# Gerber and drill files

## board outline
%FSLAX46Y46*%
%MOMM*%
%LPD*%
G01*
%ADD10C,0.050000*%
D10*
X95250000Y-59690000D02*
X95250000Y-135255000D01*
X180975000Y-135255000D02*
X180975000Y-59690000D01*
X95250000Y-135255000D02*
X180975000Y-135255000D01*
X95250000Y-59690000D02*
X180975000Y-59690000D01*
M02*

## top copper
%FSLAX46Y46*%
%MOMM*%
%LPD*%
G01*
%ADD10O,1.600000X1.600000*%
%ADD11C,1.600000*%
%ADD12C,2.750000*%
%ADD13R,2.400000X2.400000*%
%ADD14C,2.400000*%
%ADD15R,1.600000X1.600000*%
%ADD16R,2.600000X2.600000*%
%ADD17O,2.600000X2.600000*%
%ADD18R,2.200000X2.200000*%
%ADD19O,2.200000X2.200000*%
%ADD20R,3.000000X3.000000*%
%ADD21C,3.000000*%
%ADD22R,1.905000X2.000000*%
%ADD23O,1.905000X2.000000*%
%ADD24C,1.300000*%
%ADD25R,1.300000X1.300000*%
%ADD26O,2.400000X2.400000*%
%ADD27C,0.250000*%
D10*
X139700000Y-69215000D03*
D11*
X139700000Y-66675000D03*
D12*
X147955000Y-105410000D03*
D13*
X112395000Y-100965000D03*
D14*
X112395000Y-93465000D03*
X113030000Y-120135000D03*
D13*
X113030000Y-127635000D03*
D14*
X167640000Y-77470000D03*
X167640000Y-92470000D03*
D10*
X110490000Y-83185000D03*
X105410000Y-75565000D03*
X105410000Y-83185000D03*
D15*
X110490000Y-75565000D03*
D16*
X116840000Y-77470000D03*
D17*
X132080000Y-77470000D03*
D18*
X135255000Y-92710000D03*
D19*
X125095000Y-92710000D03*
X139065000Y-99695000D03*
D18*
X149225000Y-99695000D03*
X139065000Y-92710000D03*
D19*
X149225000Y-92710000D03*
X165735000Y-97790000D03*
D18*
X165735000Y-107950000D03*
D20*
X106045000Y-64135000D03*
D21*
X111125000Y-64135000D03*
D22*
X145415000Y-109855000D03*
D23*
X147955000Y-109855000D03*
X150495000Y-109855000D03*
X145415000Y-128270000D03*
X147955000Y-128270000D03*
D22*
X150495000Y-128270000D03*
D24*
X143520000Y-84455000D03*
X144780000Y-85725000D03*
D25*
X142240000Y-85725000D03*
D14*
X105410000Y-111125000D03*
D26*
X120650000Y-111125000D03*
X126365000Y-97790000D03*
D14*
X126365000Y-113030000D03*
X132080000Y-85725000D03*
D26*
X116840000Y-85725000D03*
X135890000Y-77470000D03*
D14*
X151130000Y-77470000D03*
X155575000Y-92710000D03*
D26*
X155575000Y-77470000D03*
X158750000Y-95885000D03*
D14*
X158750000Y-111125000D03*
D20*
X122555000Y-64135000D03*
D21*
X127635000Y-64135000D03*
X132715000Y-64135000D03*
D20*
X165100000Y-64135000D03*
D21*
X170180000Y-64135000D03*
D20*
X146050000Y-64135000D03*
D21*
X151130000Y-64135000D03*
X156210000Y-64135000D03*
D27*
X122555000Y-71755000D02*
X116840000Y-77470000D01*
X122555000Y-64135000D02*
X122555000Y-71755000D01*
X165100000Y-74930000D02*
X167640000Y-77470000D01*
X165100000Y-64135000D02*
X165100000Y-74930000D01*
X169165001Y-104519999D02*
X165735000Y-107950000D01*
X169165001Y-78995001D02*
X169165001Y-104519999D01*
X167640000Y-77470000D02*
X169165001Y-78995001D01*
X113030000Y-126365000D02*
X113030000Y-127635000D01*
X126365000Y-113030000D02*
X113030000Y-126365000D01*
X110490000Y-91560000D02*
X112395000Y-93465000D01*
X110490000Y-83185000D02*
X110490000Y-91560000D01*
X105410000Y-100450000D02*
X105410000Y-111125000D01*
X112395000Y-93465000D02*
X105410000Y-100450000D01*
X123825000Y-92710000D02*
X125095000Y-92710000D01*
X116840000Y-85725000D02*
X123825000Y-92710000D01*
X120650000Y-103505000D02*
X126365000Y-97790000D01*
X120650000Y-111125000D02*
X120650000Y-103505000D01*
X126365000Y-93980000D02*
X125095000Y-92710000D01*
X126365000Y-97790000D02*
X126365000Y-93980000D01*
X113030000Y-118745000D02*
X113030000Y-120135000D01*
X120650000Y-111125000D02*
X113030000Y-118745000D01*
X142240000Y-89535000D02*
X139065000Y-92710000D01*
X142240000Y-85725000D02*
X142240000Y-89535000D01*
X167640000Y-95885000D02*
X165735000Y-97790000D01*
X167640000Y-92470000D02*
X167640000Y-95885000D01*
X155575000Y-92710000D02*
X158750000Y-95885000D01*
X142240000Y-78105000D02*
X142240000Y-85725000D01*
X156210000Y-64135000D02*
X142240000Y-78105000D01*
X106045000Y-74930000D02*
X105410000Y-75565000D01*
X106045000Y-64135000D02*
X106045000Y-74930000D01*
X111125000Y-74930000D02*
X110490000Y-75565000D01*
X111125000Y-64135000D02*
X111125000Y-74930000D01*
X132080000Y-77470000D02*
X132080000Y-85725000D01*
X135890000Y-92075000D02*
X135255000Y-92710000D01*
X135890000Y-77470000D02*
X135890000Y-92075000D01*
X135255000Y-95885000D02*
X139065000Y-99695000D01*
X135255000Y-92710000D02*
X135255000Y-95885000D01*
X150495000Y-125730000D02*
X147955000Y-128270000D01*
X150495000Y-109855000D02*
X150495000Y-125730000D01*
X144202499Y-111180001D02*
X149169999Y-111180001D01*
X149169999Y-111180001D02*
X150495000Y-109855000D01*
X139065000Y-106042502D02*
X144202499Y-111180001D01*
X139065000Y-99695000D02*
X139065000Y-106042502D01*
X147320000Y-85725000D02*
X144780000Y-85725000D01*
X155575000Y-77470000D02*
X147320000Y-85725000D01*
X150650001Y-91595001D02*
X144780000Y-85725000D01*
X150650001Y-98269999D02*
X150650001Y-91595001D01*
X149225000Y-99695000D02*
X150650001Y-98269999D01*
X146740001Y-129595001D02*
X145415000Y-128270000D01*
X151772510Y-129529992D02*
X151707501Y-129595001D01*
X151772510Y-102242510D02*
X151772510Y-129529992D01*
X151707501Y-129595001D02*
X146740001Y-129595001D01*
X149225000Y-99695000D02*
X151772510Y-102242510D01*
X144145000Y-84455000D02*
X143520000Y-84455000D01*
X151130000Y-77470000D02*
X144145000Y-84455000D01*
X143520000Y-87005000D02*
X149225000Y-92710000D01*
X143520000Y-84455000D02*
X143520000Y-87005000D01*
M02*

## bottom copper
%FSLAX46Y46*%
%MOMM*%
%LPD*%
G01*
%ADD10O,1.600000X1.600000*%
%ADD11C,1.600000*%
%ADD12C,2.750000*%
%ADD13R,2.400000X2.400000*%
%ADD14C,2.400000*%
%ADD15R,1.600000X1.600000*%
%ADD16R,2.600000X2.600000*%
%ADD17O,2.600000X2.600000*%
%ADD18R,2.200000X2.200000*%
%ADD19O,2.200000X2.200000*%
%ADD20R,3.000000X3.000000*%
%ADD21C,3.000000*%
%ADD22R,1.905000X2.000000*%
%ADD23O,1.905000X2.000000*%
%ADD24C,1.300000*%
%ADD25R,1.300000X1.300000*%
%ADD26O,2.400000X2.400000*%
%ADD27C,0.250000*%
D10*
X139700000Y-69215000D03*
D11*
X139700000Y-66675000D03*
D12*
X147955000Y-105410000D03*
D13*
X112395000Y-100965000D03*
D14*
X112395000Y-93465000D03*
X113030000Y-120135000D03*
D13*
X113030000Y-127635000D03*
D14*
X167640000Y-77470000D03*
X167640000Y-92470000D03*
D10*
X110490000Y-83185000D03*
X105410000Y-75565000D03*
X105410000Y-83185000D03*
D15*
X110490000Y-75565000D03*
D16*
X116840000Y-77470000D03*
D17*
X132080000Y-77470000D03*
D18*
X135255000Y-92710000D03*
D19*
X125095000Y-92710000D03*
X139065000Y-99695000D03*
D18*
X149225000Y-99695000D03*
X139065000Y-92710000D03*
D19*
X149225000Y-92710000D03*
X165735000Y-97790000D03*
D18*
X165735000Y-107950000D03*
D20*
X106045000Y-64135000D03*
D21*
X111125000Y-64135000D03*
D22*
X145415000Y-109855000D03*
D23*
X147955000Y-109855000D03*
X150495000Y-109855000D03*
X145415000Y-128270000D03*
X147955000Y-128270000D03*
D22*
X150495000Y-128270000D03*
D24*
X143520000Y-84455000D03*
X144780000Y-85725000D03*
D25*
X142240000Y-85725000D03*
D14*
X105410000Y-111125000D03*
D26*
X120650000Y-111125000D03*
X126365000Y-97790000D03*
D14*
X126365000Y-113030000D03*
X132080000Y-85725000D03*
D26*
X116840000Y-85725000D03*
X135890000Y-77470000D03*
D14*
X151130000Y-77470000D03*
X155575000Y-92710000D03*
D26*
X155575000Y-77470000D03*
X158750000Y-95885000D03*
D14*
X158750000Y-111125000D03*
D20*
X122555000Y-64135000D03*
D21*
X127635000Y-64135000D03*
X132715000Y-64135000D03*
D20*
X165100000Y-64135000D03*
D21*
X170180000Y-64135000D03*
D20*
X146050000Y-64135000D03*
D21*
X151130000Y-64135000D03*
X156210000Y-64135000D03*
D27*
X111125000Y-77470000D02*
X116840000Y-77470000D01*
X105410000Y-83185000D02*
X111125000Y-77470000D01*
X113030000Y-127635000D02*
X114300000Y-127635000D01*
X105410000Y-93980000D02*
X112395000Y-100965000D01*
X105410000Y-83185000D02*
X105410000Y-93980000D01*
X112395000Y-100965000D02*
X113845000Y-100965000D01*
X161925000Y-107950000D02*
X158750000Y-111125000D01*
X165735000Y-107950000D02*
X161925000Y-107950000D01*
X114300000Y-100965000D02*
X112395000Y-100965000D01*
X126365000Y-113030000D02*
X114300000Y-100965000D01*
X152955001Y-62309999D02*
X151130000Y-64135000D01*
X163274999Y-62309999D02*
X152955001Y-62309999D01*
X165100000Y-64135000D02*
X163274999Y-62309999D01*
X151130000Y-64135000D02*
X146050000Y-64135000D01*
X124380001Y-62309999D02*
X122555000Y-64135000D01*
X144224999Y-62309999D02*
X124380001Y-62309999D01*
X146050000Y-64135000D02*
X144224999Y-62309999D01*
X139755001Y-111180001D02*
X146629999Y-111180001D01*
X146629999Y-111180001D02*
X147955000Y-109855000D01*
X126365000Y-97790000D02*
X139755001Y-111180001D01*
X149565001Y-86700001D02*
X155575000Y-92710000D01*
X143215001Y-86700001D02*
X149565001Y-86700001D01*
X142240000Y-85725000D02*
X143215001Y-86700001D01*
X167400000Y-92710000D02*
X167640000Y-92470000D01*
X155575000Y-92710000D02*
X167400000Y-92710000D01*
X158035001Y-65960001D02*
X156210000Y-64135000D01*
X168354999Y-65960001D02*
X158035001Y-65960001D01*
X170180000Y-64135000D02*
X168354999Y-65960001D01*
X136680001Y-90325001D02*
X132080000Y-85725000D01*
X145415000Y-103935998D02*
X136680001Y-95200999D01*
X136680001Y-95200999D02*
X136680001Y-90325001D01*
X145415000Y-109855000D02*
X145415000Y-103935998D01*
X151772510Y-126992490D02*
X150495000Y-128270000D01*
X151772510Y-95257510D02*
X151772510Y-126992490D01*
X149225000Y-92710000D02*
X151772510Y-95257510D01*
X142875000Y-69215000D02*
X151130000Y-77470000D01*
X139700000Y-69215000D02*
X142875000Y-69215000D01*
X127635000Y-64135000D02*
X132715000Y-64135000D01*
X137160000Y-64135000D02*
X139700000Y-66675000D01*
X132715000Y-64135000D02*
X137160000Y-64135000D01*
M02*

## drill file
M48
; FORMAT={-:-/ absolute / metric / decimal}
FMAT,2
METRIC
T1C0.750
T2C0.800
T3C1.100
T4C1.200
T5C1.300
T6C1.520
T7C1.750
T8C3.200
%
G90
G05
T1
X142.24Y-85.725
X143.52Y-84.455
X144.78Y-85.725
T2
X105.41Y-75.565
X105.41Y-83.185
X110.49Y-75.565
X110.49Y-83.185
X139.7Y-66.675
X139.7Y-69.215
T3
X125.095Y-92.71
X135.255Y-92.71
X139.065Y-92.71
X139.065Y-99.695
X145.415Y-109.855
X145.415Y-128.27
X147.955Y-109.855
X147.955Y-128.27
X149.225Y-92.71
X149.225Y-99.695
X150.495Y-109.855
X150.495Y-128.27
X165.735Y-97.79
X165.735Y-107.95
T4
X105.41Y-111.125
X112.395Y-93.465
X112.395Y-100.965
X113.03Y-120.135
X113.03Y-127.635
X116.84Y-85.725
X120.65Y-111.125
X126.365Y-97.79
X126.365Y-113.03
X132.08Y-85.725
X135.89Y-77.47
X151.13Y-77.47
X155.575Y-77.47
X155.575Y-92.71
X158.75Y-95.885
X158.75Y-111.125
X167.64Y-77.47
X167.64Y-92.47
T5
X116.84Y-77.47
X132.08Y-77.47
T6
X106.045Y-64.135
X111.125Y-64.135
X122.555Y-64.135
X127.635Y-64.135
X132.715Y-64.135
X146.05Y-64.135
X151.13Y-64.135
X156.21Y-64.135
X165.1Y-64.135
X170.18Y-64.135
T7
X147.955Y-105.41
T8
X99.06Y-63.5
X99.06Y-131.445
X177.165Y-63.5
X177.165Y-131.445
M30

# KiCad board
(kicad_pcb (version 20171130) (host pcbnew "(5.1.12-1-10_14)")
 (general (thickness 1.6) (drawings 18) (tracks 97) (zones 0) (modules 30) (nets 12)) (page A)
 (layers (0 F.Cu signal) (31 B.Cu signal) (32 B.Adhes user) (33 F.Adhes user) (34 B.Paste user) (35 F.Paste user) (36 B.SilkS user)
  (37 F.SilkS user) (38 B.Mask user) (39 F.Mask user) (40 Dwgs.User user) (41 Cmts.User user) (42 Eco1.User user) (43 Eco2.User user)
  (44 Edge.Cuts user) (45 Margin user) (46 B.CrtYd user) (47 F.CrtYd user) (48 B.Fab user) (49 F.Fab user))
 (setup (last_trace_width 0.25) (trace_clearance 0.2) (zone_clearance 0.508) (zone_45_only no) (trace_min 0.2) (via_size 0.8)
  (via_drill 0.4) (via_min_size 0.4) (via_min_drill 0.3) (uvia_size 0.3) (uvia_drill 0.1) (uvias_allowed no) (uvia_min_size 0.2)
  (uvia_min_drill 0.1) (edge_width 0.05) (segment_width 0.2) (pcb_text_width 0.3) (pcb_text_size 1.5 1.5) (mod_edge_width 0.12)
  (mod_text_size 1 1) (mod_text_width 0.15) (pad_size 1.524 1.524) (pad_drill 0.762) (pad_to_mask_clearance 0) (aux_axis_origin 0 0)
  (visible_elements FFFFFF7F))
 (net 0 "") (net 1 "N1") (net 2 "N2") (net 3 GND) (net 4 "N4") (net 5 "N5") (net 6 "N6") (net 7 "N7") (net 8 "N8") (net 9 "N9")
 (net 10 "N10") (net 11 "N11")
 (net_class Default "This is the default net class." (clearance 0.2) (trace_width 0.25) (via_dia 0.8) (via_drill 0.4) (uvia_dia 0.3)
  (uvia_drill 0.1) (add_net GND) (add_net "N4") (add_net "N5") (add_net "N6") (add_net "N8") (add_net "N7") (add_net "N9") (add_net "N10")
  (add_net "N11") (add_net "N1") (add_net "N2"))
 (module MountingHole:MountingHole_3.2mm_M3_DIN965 (layer F.Cu) (at 177.165 131.445)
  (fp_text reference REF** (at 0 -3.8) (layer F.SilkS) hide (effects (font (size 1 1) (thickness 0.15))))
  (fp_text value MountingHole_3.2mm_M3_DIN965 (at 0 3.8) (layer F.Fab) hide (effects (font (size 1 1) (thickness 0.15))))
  (pad 1 np_thru_hole circle (at 0 0) (size 3.2 3.2) (drill 3.2) (layers *.Cu *.Mask)))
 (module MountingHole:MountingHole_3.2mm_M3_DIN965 (layer F.Cu) (at 99.06 131.445)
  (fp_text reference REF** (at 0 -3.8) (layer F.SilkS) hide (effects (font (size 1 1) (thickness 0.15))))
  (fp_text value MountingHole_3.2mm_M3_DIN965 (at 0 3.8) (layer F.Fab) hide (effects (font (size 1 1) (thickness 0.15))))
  (pad 1 np_thru_hole circle (at 0 0) (size 3.2 3.2) (drill 3.2) (layers *.Cu *.Mask)))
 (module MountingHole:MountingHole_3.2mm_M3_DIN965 (layer F.Cu) (at 99.06 63.5)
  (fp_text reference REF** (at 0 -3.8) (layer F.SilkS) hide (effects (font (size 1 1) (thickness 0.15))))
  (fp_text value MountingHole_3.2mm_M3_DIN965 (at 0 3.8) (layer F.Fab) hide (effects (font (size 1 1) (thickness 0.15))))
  (pad 1 np_thru_hole circle (at 0 0) (size 3.2 3.2) (drill 3.2) (layers *.Cu *.Mask)))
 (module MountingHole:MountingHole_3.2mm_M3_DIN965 (layer F.Cu) (at 177.165 63.5)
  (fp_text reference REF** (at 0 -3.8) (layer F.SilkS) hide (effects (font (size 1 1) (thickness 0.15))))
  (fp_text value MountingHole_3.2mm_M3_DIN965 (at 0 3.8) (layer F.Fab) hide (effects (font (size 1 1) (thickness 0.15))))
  (pad 1 np_thru_hole circle (at 0 0) (size 3.2 3.2) (drill 3.2) (layers *.Cu *.Mask)))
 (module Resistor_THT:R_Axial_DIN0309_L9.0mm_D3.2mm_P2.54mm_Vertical (layer F.Cu) (at 139.7 66.675 270)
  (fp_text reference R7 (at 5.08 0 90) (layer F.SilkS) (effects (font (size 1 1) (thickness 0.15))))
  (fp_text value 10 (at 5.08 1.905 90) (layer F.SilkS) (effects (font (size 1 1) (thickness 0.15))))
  (pad 2 thru_hole oval (at 2.54 0 270) (size 1.6 1.6) (drill 0.8) (layers *.Cu *.Mask) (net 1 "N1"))
  (pad 1 thru_hole circle (at 0 0 270) (size 1.6 1.6) (drill 0.8) (layers *.Cu *.Mask) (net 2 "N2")))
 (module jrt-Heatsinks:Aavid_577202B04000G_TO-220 (layer F.Cu) (at 147.955 105.41 180)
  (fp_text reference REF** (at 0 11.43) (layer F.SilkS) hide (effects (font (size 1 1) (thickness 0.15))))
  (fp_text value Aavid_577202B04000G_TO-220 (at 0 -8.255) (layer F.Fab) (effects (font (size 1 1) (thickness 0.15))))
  (pad "" thru_hole circle (at 0 0 180) (size 2.75 2.75) (drill 1.75) (layers *.Cu *.Mask)))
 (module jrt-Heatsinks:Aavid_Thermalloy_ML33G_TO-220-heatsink (layer F.Cu) (at 167.005 135.255 180)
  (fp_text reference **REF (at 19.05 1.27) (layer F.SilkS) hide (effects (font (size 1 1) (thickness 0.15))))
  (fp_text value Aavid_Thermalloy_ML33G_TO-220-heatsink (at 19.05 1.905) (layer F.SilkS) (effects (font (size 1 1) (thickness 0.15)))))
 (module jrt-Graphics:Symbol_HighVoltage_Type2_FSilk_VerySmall (layer F.Cu) (at 168.91 112.395 90)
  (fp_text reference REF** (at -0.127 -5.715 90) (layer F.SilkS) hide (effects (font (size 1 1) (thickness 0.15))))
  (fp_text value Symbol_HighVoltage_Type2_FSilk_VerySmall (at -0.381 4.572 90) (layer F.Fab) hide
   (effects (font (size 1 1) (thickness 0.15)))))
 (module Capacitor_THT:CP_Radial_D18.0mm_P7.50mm (layer F.Cu) (at 112.395 100.965 90)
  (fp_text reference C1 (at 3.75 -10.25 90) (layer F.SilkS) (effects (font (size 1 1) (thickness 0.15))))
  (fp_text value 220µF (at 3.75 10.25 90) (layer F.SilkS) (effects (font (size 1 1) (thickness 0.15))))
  (pad 1 thru_hole rect (at 0 0 90) (size 2.4 2.4) (drill 1.2) (layers *.Cu *.Mask) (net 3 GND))
  (pad 2 thru_hole circle (at 7.5 0 90) (size 2.4 2.4) (drill 1.2) (layers *.Cu *.Mask) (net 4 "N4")))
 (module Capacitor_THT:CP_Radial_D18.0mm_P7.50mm (layer F.Cu) (at 113.03 127.635 90)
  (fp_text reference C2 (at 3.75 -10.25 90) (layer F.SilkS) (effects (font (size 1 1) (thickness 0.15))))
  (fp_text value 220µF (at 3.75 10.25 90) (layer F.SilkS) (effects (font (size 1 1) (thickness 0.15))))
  (pad 2 thru_hole circle (at 7.5 0 90) (size 2.4 2.4) (drill 1.2) (layers *.Cu *.Mask) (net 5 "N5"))
  (pad 1 thru_hole rect (at 0 0 90) (size 2.4 2.4) (drill 1.2) (layers *.Cu *.Mask) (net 3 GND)))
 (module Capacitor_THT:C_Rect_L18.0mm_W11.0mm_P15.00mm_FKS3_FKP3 (layer F.Cu) (at 167.64 77.47 270)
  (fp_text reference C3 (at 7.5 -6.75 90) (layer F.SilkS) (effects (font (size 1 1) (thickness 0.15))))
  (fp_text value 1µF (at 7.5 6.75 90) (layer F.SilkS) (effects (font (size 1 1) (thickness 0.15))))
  (pad 1 thru_hole circle (at 0 0 270) (size 2.4 2.4) (drill 1.2) (layers *.Cu *.Mask) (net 3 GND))
  (pad 2 thru_hole circle (at 15 0 270) (size 2.4 2.4) (drill 1.2) (layers *.Cu *.Mask) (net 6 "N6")))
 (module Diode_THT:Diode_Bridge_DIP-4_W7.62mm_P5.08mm (layer F.Cu) (at 110.49 75.565 270)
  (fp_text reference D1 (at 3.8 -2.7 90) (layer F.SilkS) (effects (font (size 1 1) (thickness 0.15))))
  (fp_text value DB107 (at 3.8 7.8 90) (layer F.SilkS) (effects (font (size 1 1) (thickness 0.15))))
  (pad 4 thru_hole oval (at 7.62 0 270) (size 1.6 1.6) (drill 0.8) (layers *.Cu *.Mask) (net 4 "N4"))
  (pad 2 thru_hole oval (at 0 5.08 270) (size 1.6 1.6) (drill 0.8) (layers *.Cu *.Mask) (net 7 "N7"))
  (pad 3 thru_hole oval (at 7.62 5.08 270) (size 1.6 1.6) (drill 0.8) (layers *.Cu *.Mask) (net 3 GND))
  (pad 1 thru_hole rect (at 0 0 270) (size 1.6 1.6) (drill 0.8) (layers *.Cu *.Mask) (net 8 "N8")))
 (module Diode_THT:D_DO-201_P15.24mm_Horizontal (layer F.Cu) (at 116.84 77.47)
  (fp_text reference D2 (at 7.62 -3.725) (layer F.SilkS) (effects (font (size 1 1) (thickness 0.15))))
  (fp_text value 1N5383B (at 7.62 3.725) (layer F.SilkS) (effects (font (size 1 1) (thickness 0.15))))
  (pad 1 thru_hole rect (at 0 0) (size 2.6 2.6) (drill 1.3) (layers *.Cu *.Mask) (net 3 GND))
  (pad 2 thru_hole oval (at 15.24 0) (size 2.6 2.6) (drill 1.3) (layers *.Cu *.Mask) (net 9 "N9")))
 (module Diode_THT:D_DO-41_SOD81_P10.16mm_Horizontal (layer F.Cu) (at 135.255 92.71 180)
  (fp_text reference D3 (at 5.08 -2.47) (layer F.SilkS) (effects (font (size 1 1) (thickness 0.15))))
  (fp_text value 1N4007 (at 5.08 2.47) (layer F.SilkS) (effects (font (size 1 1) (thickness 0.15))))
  (pad 1 thru_hole rect (at 0 0 180) (size 2.2 2.2) (drill 1.1) (layers *.Cu *.Mask) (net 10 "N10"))
  (pad 2 thru_hole oval (at 10.16 0 180) (size 2.2 2.2) (drill 1.1) (layers *.Cu *.Mask) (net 5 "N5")))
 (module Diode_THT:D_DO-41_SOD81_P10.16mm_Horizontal (layer F.Cu) (at 149.225 99.695 180)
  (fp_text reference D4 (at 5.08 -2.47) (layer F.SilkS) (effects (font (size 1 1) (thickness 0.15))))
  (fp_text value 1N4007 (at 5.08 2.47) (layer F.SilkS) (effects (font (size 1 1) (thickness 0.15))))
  (pad 2 thru_hole oval (at 10.16 0 180) (size 2.2 2.2) (drill 1.1) (layers *.Cu *.Mask) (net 10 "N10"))
  (pad 1 thru_hole rect (at 0 0 180) (size 2.2 2.2) (drill 1.1) (layers *.Cu *.Mask) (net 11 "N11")))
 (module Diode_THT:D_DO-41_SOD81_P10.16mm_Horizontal (layer F.Cu) (at 139.065 92.71)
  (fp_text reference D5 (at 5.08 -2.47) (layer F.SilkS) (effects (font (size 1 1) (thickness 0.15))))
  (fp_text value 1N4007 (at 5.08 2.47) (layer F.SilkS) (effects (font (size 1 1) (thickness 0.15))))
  (pad 1 thru_hole rect (at 0 0) (size 2.2 2.2) (drill 1.1) (layers *.Cu *.Mask) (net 6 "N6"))
  (pad 2 thru_hole oval (at 10.16 0) (size 2.2 2.2) (drill 1.1) (layers *.Cu *.Mask) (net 1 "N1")))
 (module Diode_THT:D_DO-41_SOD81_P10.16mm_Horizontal (layer F.Cu) (at 165.735 107.95 90)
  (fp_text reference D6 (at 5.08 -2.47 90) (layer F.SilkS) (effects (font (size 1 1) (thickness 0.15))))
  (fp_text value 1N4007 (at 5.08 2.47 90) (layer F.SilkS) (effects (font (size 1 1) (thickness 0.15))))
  (pad 2 thru_hole oval (at 10.16 0 90) (size 2.2 2.2) (drill 1.1) (layers *.Cu *.Mask) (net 6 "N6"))
  (pad 1 thru_hole rect (at 0 0 90) (size 2.2 2.2) (drill 1.1) (layers *.Cu *.Mask) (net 3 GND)))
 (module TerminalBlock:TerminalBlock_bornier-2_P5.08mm (layer F.Cu) (at 106.045 64.135)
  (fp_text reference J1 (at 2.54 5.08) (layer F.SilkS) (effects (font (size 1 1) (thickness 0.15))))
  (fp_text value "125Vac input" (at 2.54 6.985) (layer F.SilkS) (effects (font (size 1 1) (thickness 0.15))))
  (pad 1 thru_hole rect (at 0 0) (size 3 3) (drill 1.52) (layers *.Cu *.Mask) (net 7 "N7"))
  (pad 2 thru_hole circle (at 5.08 0) (size 3 3) (drill 1.52) (layers *.Cu *.Mask) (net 8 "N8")))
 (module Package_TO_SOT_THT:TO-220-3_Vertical (layer F.Cu) (at 145.415 109.855)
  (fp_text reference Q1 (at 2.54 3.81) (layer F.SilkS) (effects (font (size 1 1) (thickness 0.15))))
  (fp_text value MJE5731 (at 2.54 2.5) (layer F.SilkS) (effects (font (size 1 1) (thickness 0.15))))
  (pad 1 thru_hole rect (at 0 0) (size 1.905 2) (drill 1.1) (layers *.Cu *.Mask) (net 9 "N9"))
  (pad 2 thru_hole oval (at 2.54 0) (size 1.905 2) (drill 1.1) (layers *.Cu *.Mask) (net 5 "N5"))
  (pad 3 thru_hole oval (at 5.08 0) (size 1.905 2) (drill 1.1) (layers *.Cu *.Mask) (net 10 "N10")))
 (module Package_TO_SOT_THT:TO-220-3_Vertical (layer F.Cu) (at 150.495 128.27 180)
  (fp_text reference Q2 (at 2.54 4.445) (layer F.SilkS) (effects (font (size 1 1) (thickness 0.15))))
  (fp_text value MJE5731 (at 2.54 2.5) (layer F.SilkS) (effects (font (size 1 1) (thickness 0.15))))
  (pad 3 thru_hole oval (at 5.08 0 180) (size 1.905 2) (drill 1.1) (layers *.Cu *.Mask) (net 11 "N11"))
  (pad 2 thru_hole oval (at 2.54 0 180) (size 1.905 2) (drill 1.1) (layers *.Cu *.Mask) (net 10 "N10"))
  (pad 1 thru_hole rect (at 0 0 180) (size 1.905 2) (drill 1.1) (layers *.Cu *.Mask) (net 1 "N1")))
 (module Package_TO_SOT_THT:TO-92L (layer F.Cu) (at 142.24 85.725)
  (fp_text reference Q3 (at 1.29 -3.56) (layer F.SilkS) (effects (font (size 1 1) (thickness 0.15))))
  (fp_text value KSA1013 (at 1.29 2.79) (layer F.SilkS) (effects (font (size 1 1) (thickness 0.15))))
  (pad 2 thru_hole circle (at 1.28 -1.27) (size 1.3 1.3) (drill 0.75) (layers *.Cu *.Mask) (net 1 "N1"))
  (pad 3 thru_hole circle (at 2.54 0) (size 1.3 1.3) (drill 0.75) (layers *.Cu *.Mask) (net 11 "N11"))
  (pad 1 thru_hole rect (at 0 0) (size 1.3 1.3) (drill 0.75) (layers *.Cu *.Mask) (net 6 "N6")))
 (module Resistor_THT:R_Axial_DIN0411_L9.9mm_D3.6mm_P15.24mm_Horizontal (layer F.Cu) (at 105.41 111.125)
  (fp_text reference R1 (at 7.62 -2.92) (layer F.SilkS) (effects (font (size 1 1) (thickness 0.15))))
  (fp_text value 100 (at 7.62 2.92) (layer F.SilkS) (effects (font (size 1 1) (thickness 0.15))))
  (pad 1 thru_hole circle (at 0 0) (size 2.4 2.4) (drill 1.2) (layers *.Cu *.Mask) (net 4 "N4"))
  (pad 2 thru_hole oval (at 15.24 0) (size 2.4 2.4) (drill 1.2) (layers *.Cu *.Mask) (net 5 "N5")))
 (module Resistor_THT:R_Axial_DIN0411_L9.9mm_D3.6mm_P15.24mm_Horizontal (layer F.Cu) (at 126.365 113.03 90)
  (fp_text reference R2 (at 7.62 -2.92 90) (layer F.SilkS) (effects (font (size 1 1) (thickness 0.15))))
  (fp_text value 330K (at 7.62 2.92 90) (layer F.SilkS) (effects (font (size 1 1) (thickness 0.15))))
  (pad 2 thru_hole oval (at 15.24 0 90) (size 2.4 2.4) (drill 1.2) (layers *.Cu *.Mask) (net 5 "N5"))
  (pad 1 thru_hole circle (at 0 0 90) (size 2.4 2.4) (drill 1.2) (layers *.Cu *.Mask) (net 3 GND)))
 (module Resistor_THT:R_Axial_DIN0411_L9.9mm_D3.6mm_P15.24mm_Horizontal (layer F.Cu) (at 132.08 85.725 180)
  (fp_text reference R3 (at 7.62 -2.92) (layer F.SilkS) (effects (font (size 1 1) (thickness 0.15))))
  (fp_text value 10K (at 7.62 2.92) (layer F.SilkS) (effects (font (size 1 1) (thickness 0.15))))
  (pad 1 thru_hole circle (at 0 0 180) (size 2.4 2.4) (drill 1.2) (layers *.Cu *.Mask) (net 9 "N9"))
  (pad 2 thru_hole oval (at 15.24 0 180) (size 2.4 2.4) (drill 1.2) (layers *.Cu *.Mask) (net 5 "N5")))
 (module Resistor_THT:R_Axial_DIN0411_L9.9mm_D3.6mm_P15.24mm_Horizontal (layer F.Cu) (at 151.13 77.47 180)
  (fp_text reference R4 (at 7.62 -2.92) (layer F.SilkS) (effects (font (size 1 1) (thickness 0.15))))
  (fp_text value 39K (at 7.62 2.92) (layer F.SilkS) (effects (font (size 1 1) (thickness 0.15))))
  (pad 2 thru_hole oval (at 15.24 0 180) (size 2.4 2.4) (drill 1.2) (layers *.Cu *.Mask) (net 10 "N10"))
  (pad 1 thru_hole circle (at 0 0 180) (size 2.4 2.4) (drill 1.2) (layers *.Cu *.Mask) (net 1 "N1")))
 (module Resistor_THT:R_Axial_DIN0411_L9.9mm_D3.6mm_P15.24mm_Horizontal (layer F.Cu) (at 155.575 92.71 90)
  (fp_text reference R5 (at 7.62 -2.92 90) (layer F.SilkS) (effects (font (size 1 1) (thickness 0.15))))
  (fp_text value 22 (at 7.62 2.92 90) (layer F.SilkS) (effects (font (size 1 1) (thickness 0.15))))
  (pad 1 thru_hole circle (at 0 0 90) (size 2.4 2.4) (drill 1.2) (layers *.Cu *.Mask) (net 6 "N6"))
  (pad 2 thru_hole oval (at 15.24 0 90) (size 2.4 2.4) (drill 1.2) (layers *.Cu *.Mask) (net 11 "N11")))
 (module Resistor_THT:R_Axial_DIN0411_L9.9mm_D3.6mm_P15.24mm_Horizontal (layer F.Cu) (at 158.75 111.125 90)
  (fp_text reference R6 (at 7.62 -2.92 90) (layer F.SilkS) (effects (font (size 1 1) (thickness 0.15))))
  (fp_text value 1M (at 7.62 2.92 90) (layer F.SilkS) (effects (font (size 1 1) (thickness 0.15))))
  (pad 2 thru_hole oval (at 15.24 0 90) (size 2.4 2.4) (drill 1.2) (layers *.Cu *.Mask) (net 6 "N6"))
  (pad 1 thru_hole circle (at 0 0 90) (size 2.4 2.4) (drill 1.2) (layers *.Cu *.Mask) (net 3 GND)))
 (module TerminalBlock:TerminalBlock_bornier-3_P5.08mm (layer F.Cu) (at 122.555 64.135)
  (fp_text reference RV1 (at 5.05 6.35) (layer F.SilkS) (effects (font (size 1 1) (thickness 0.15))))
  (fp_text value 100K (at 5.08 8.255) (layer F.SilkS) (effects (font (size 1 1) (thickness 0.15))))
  (pad 1 thru_hole rect (at 0 0) (size 3 3) (drill 1.52) (layers *.Cu *.Mask) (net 3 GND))
  (pad 2 thru_hole circle (at 5.08 0) (size 3 3) (drill 1.52) (layers *.Cu *.Mask) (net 2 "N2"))
  (pad 3 thru_hole circle (at 10.16 0) (size 3 3) (drill 1.52) (layers *.Cu *.Mask) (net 2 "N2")))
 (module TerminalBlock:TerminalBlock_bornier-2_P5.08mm (layer F.Cu) (at 165.1 64.135)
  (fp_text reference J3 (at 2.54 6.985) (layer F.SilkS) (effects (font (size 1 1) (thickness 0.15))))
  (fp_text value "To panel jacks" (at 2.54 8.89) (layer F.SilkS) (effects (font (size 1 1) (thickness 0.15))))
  (pad 1 thru_hole rect (at 0 0) (size 3 3) (drill 1.52) (layers *.Cu *.Mask) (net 3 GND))
  (pad 2 thru_hole circle (at 5.08 0) (size 3 3) (drill 1.52) (layers *.Cu *.Mask) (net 6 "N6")))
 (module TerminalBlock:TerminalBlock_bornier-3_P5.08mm (layer F.Cu) (at 146.05 64.135)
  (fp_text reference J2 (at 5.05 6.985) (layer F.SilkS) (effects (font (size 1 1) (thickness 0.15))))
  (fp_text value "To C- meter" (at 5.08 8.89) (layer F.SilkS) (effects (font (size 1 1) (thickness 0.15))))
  (pad 1 thru_hole rect (at 0 0) (size 3 3) (drill 1.52) (layers *.Cu *.Mask) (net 3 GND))
  (pad 2 thru_hole circle (at 5.08 0) (size 3 3) (drill 1.52) (layers *.Cu *.Mask) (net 3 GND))
  (pad 3 thru_hole circle (at 10.16 0) (size 3 3) (drill 1.52) (layers *.Cu *.Mask) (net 6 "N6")))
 (gr_line (start 95.25 59.69) (end 95.25 135.255) (layer Edge.Cuts) (width 0.05))
 (gr_line (start 180.975 135.255) (end 180.975 59.69) (layer Edge.Cuts) (width 0.05))
 (gr_line (start 95.25 135.255) (end 180.975 135.255) (layer Edge.Cuts) (width 0.05))
 (gr_line (start 95.25 59.69) (end 180.975 59.69) (layer Edge.Cuts) (width 0.05))
 (segment (start 122.555 71.755) (end 116.84 77.47) (width 0.25) (layer F.Cu) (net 3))
 (segment (start 122.555 64.135) (end 122.555 71.755) (width 0.25) (layer F.Cu) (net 3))
 (segment (start 111.125 77.47) (end 116.84 77.47) (width 0.25) (layer B.Cu) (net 3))
 (segment (start 105.41 83.185) (end 111.125 77.47) (width 0.25) (layer B.Cu) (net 3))
 (segment (start 165.1 74.93) (end 167.64 77.47) (width 0.25) (layer F.Cu) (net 3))
 (segment (start 165.1 64.135) (end 165.1 74.93) (width 0.25) (layer F.Cu) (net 3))
 (segment (start 113.03 127.635) (end 114.3 127.635) (width 0.25) (layer B.Cu) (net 3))
 (segment (start 105.41 93.98) (end 112.395 100.965) (width 0.25) (layer B.Cu) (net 3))
 (segment (start 105.41 83.185) (end 105.41 93.98) (width 0.25) (layer B.Cu) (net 3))
 (segment (start 112.395 100.965) (end 113.845 100.965) (width 0.25) (layer B.Cu) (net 3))
 (segment (start 169.165001 104.519999) (end 165.735 107.95) (width 0.25) (layer F.Cu) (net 3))
 (segment (start 169.165001 78.995001) (end 169.165001 104.519999) (width 0.25) (layer F.Cu) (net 3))
 (segment (start 167.64 77.47) (end 169.165001 78.995001) (width 0.25) (layer F.Cu) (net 3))
 (segment (start 161.925 107.95) (end 158.75 111.125) (width 0.25) (layer B.Cu) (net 3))
 (segment (start 165.735 107.95) (end 161.925 107.95) (width 0.25) (layer B.Cu) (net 3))
 (segment (start 114.3 100.965) (end 112.395 100.965) (width 0.25) (layer B.Cu) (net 3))
 (segment (start 126.365 113.03) (end 114.3 100.965) (width 0.25) (layer B.Cu) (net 3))
 (segment (start 113.03 126.365) (end 113.03 127.635) (width 0.25) (layer F.Cu) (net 3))
 (segment (start 126.365 113.03) (end 113.03 126.365) (width 0.25) (layer F.Cu) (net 3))
 (segment (start 152.955001 62.309999) (end 151.13 64.135) (width 0.25) (layer B.Cu) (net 3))
 (segment (start 163.274999 62.309999) (end 152.955001 62.309999) (width 0.25) (layer B.Cu) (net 3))
 (segment (start 165.1 64.135) (end 163.274999 62.309999) (width 0.25) (layer B.Cu) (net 3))
 (segment (start 151.13 64.135) (end 146.05 64.135) (width 0.25) (layer B.Cu) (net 3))
 (segment (start 124.380001 62.309999) (end 122.555 64.135) (width 0.25) (layer B.Cu) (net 3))
 (segment (start 144.224999 62.309999) (end 124.380001 62.309999) (width 0.25) (layer B.Cu) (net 3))
 (segment (start 146.05 64.135) (end 144.224999 62.309999) (width 0.25) (layer B.Cu) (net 3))
 (segment (start 110.49 91.56) (end 112.395 93.465) (width 0.25) (layer F.Cu) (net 4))
 (segment (start 110.49 83.185) (end 110.49 91.56) (width 0.25) (layer F.Cu) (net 4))
 (segment (start 105.41 100.45) (end 105.41 111.125) (width 0.25) (layer F.Cu) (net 4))
 (segment (start 112.395 93.465) (end 105.41 100.45) (width 0.25) (layer F.Cu) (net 4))
 (segment (start 123.825 92.71) (end 125.095 92.71) (width 0.25) (layer F.Cu) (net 5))
 (segment (start 116.84 85.725) (end 123.825 92.71) (width 0.25) (layer F.Cu) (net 5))
 (segment (start 120.65 103.505) (end 126.365 97.79) (width 0.25) (layer F.Cu) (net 5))
 (segment (start 120.65 111.125) (end 120.65 103.505) (width 0.25) (layer F.Cu) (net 5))
 (segment (start 126.365 93.98) (end 125.095 92.71) (width 0.25) (layer F.Cu) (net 5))
 (segment (start 126.365 97.79) (end 126.365 93.98) (width 0.25) (layer F.Cu) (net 5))
 (segment (start 139.755001 111.180001) (end 146.629999 111.180001) (width 0.25) (layer B.Cu) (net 5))
 (segment (start 146.629999 111.180001) (end 147.955 109.855) (width 0.25) (layer B.Cu) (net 5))
 (segment (start 126.365 97.79) (end 139.755001 111.180001) (width 0.25) (layer B.Cu) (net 5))
 (segment (start 113.03 118.745) (end 113.03 120.135) (width 0.25) (layer F.Cu) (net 5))
 (segment (start 120.65 111.125) (end 113.03 118.745) (width 0.25) (layer F.Cu) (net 5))
 (segment (start 142.24 89.535) (end 139.065 92.71) (width 0.25) (layer F.Cu) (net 6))
 (segment (start 142.24 85.725) (end 142.24 89.535) (width 0.25) (layer F.Cu) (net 6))
 (segment (start 149.565001 86.700001) (end 155.575 92.71) (width 0.25) (layer B.Cu) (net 6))
 (segment (start 143.215001 86.700001) (end 149.565001 86.700001) (width 0.25) (layer B.Cu) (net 6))
 (segment (start 142.24 85.725) (end 143.215001 86.700001) (width 0.25) (layer B.Cu) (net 6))
 (segment (start 167.4 92.71) (end 167.64 92.47) (width 0.25) (layer B.Cu) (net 6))
 (segment (start 155.575 92.71) (end 167.4 92.71) (width 0.25) (layer B.Cu) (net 6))
 (segment (start 167.64 95.885) (end 165.735 97.79) (width 0.25) (layer F.Cu) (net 6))
 (segment (start 167.64 92.47) (end 167.64 95.885) (width 0.25) (layer F.Cu) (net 6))
 (segment (start 155.575 92.71) (end 158.75 95.885) (width 0.25) (layer F.Cu) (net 6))
 (segment (start 142.24 78.105) (end 142.24 85.725) (width 0.25) (layer F.Cu) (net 6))
 (segment (start 156.21 64.135) (end 142.24 78.105) (width 0.25) (layer F.Cu) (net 6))
 (segment (start 158.035001 65.960001) (end 156.21 64.135) (width 0.25) (layer B.Cu) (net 6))
 (segment (start 168.354999 65.960001) (end 158.035001 65.960001) (width 0.25) (layer B.Cu) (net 6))
 (segment (start 170.18 64.135) (end 168.354999 65.960001) (width 0.25) (layer B.Cu) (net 6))
 (segment (start 106.045 74.93) (end 105.41 75.565) (width 0.25) (layer F.Cu) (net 7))
 (segment (start 106.045 64.135) (end 106.045 74.93) (width 0.25) (layer F.Cu) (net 7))
 (segment (start 111.125 74.93) (end 110.49 75.565) (width 0.25) (layer F.Cu) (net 8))
 (segment (start 111.125 64.135) (end 111.125 74.93) (width 0.25) (layer F.Cu) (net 8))
 (segment (start 132.08 77.47) (end 132.08 85.725) (width 0.25) (layer F.Cu) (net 9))
 (segment (start 136.680001 90.325001) (end 132.08 85.725) (width 0.25) (layer B.Cu) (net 9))
 (segment (start 145.415 103.935998) (end 136.680001 95.200999) (width 0.25) (layer B.Cu) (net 9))
 (segment (start 136.680001 95.200999) (end 136.680001 90.325001) (width 0.25) (layer B.Cu) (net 9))
 (segment (start 145.415 109.855) (end 145.415 103.935998) (width 0.25) (layer B.Cu) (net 9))
 (segment (start 135.89 92.075) (end 135.255 92.71) (width 0.25) (layer F.Cu) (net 10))
 (segment (start 135.89 77.47) (end 135.89 92.075) (width 0.25) (layer F.Cu) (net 10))
 (segment (start 135.255 95.885) (end 139.065 99.695) (width 0.25) (layer F.Cu) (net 10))
 (segment (start 135.255 92.71) (end 135.255 95.885) (width 0.25) (layer F.Cu) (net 10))
 (segment (start 150.495 125.73) (end 147.955 128.27) (width 0.25) (layer F.Cu) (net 10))
 (segment (start 150.495 109.855) (end 150.495 125.73) (width 0.25) (layer F.Cu) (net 10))
 (segment (start 144.202499 111.180001) (end 149.169999 111.180001) (width 0.25) (layer F.Cu) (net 10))
 (segment (start 149.169999 111.180001) (end 150.495 109.855) (width 0.25) (layer F.Cu) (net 10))
 (segment (start 139.065 106.042502) (end 144.202499 111.180001) (width 0.25) (layer F.Cu) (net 10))
 (segment (start 139.065 99.695) (end 139.065 106.042502) (width 0.25) (layer F.Cu) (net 10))
 (segment (start 147.32 85.725) (end 144.78 85.725) (width 0.25) (layer F.Cu) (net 11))
 (segment (start 155.575 77.47) (end 147.32 85.725) (width 0.25) (layer F.Cu) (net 11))
 (segment (start 150.650001 91.595001) (end 144.78 85.725) (width 0.25) (layer F.Cu) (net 11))
 (segment (start 150.650001 98.269999) (end 150.650001 91.595001) (width 0.25) (layer F.Cu) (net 11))
 (segment (start 149.225 99.695) (end 150.650001 98.269999) (width 0.25) (layer F.Cu) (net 11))
 (segment (start 146.740001 129.595001) (end 145.415 128.27) (width 0.25) (layer F.Cu) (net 11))
 (segment (start 151.77251 129.529992) (end 151.707501 129.595001) (width 0.25) (layer F.Cu) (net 11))
 (segment (start 151.77251 102.24251) (end 151.77251 129.529992) (width 0.25) (layer F.Cu) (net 11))
 (segment (start 151.707501 129.595001) (end 146.740001 129.595001) (width 0.25) (layer F.Cu) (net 11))
 (segment (start 149.225 99.695) (end 151.77251 102.24251) (width 0.25) (layer F.Cu) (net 11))
 (segment (start 144.145 84.455) (end 143.52 84.455) (width 0.25) (layer F.Cu) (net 1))
 (segment (start 151.13 77.47) (end 144.145 84.455) (width 0.25) (layer F.Cu) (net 1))
 (segment (start 143.52 87.005) (end 149.225 92.71) (width 0.25) (layer F.Cu) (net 1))
 (segment (start 143.52 84.455) (end 143.52 87.005) (width 0.25) (layer F.Cu) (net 1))
 (segment (start 151.77251 126.99249) (end 150.495 128.27) (width 0.25) (layer B.Cu) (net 1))
 (segment (start 151.77251 95.25751) (end 151.77251 126.99249) (width 0.25) (layer B.Cu) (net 1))
 (segment (start 149.225 92.71) (end 151.77251 95.25751) (width 0.25) (layer B.Cu) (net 1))
 (segment (start 142.875 69.215) (end 151.13 77.47) (width 0.25) (layer B.Cu) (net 1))
 (segment (start 139.7 69.215) (end 142.875 69.215) (width 0.25) (layer B.Cu) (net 1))
 (segment (start 127.635 64.135) (end 132.715 64.135) (width 0.25) (layer B.Cu) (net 2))
 (segment (start 137.16 64.135) (end 139.7 66.675) (width 0.25) (layer B.Cu) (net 2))
 (segment (start 132.715 64.135) (end 137.16 64.135) (width 0.25) (layer B.Cu) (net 2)))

